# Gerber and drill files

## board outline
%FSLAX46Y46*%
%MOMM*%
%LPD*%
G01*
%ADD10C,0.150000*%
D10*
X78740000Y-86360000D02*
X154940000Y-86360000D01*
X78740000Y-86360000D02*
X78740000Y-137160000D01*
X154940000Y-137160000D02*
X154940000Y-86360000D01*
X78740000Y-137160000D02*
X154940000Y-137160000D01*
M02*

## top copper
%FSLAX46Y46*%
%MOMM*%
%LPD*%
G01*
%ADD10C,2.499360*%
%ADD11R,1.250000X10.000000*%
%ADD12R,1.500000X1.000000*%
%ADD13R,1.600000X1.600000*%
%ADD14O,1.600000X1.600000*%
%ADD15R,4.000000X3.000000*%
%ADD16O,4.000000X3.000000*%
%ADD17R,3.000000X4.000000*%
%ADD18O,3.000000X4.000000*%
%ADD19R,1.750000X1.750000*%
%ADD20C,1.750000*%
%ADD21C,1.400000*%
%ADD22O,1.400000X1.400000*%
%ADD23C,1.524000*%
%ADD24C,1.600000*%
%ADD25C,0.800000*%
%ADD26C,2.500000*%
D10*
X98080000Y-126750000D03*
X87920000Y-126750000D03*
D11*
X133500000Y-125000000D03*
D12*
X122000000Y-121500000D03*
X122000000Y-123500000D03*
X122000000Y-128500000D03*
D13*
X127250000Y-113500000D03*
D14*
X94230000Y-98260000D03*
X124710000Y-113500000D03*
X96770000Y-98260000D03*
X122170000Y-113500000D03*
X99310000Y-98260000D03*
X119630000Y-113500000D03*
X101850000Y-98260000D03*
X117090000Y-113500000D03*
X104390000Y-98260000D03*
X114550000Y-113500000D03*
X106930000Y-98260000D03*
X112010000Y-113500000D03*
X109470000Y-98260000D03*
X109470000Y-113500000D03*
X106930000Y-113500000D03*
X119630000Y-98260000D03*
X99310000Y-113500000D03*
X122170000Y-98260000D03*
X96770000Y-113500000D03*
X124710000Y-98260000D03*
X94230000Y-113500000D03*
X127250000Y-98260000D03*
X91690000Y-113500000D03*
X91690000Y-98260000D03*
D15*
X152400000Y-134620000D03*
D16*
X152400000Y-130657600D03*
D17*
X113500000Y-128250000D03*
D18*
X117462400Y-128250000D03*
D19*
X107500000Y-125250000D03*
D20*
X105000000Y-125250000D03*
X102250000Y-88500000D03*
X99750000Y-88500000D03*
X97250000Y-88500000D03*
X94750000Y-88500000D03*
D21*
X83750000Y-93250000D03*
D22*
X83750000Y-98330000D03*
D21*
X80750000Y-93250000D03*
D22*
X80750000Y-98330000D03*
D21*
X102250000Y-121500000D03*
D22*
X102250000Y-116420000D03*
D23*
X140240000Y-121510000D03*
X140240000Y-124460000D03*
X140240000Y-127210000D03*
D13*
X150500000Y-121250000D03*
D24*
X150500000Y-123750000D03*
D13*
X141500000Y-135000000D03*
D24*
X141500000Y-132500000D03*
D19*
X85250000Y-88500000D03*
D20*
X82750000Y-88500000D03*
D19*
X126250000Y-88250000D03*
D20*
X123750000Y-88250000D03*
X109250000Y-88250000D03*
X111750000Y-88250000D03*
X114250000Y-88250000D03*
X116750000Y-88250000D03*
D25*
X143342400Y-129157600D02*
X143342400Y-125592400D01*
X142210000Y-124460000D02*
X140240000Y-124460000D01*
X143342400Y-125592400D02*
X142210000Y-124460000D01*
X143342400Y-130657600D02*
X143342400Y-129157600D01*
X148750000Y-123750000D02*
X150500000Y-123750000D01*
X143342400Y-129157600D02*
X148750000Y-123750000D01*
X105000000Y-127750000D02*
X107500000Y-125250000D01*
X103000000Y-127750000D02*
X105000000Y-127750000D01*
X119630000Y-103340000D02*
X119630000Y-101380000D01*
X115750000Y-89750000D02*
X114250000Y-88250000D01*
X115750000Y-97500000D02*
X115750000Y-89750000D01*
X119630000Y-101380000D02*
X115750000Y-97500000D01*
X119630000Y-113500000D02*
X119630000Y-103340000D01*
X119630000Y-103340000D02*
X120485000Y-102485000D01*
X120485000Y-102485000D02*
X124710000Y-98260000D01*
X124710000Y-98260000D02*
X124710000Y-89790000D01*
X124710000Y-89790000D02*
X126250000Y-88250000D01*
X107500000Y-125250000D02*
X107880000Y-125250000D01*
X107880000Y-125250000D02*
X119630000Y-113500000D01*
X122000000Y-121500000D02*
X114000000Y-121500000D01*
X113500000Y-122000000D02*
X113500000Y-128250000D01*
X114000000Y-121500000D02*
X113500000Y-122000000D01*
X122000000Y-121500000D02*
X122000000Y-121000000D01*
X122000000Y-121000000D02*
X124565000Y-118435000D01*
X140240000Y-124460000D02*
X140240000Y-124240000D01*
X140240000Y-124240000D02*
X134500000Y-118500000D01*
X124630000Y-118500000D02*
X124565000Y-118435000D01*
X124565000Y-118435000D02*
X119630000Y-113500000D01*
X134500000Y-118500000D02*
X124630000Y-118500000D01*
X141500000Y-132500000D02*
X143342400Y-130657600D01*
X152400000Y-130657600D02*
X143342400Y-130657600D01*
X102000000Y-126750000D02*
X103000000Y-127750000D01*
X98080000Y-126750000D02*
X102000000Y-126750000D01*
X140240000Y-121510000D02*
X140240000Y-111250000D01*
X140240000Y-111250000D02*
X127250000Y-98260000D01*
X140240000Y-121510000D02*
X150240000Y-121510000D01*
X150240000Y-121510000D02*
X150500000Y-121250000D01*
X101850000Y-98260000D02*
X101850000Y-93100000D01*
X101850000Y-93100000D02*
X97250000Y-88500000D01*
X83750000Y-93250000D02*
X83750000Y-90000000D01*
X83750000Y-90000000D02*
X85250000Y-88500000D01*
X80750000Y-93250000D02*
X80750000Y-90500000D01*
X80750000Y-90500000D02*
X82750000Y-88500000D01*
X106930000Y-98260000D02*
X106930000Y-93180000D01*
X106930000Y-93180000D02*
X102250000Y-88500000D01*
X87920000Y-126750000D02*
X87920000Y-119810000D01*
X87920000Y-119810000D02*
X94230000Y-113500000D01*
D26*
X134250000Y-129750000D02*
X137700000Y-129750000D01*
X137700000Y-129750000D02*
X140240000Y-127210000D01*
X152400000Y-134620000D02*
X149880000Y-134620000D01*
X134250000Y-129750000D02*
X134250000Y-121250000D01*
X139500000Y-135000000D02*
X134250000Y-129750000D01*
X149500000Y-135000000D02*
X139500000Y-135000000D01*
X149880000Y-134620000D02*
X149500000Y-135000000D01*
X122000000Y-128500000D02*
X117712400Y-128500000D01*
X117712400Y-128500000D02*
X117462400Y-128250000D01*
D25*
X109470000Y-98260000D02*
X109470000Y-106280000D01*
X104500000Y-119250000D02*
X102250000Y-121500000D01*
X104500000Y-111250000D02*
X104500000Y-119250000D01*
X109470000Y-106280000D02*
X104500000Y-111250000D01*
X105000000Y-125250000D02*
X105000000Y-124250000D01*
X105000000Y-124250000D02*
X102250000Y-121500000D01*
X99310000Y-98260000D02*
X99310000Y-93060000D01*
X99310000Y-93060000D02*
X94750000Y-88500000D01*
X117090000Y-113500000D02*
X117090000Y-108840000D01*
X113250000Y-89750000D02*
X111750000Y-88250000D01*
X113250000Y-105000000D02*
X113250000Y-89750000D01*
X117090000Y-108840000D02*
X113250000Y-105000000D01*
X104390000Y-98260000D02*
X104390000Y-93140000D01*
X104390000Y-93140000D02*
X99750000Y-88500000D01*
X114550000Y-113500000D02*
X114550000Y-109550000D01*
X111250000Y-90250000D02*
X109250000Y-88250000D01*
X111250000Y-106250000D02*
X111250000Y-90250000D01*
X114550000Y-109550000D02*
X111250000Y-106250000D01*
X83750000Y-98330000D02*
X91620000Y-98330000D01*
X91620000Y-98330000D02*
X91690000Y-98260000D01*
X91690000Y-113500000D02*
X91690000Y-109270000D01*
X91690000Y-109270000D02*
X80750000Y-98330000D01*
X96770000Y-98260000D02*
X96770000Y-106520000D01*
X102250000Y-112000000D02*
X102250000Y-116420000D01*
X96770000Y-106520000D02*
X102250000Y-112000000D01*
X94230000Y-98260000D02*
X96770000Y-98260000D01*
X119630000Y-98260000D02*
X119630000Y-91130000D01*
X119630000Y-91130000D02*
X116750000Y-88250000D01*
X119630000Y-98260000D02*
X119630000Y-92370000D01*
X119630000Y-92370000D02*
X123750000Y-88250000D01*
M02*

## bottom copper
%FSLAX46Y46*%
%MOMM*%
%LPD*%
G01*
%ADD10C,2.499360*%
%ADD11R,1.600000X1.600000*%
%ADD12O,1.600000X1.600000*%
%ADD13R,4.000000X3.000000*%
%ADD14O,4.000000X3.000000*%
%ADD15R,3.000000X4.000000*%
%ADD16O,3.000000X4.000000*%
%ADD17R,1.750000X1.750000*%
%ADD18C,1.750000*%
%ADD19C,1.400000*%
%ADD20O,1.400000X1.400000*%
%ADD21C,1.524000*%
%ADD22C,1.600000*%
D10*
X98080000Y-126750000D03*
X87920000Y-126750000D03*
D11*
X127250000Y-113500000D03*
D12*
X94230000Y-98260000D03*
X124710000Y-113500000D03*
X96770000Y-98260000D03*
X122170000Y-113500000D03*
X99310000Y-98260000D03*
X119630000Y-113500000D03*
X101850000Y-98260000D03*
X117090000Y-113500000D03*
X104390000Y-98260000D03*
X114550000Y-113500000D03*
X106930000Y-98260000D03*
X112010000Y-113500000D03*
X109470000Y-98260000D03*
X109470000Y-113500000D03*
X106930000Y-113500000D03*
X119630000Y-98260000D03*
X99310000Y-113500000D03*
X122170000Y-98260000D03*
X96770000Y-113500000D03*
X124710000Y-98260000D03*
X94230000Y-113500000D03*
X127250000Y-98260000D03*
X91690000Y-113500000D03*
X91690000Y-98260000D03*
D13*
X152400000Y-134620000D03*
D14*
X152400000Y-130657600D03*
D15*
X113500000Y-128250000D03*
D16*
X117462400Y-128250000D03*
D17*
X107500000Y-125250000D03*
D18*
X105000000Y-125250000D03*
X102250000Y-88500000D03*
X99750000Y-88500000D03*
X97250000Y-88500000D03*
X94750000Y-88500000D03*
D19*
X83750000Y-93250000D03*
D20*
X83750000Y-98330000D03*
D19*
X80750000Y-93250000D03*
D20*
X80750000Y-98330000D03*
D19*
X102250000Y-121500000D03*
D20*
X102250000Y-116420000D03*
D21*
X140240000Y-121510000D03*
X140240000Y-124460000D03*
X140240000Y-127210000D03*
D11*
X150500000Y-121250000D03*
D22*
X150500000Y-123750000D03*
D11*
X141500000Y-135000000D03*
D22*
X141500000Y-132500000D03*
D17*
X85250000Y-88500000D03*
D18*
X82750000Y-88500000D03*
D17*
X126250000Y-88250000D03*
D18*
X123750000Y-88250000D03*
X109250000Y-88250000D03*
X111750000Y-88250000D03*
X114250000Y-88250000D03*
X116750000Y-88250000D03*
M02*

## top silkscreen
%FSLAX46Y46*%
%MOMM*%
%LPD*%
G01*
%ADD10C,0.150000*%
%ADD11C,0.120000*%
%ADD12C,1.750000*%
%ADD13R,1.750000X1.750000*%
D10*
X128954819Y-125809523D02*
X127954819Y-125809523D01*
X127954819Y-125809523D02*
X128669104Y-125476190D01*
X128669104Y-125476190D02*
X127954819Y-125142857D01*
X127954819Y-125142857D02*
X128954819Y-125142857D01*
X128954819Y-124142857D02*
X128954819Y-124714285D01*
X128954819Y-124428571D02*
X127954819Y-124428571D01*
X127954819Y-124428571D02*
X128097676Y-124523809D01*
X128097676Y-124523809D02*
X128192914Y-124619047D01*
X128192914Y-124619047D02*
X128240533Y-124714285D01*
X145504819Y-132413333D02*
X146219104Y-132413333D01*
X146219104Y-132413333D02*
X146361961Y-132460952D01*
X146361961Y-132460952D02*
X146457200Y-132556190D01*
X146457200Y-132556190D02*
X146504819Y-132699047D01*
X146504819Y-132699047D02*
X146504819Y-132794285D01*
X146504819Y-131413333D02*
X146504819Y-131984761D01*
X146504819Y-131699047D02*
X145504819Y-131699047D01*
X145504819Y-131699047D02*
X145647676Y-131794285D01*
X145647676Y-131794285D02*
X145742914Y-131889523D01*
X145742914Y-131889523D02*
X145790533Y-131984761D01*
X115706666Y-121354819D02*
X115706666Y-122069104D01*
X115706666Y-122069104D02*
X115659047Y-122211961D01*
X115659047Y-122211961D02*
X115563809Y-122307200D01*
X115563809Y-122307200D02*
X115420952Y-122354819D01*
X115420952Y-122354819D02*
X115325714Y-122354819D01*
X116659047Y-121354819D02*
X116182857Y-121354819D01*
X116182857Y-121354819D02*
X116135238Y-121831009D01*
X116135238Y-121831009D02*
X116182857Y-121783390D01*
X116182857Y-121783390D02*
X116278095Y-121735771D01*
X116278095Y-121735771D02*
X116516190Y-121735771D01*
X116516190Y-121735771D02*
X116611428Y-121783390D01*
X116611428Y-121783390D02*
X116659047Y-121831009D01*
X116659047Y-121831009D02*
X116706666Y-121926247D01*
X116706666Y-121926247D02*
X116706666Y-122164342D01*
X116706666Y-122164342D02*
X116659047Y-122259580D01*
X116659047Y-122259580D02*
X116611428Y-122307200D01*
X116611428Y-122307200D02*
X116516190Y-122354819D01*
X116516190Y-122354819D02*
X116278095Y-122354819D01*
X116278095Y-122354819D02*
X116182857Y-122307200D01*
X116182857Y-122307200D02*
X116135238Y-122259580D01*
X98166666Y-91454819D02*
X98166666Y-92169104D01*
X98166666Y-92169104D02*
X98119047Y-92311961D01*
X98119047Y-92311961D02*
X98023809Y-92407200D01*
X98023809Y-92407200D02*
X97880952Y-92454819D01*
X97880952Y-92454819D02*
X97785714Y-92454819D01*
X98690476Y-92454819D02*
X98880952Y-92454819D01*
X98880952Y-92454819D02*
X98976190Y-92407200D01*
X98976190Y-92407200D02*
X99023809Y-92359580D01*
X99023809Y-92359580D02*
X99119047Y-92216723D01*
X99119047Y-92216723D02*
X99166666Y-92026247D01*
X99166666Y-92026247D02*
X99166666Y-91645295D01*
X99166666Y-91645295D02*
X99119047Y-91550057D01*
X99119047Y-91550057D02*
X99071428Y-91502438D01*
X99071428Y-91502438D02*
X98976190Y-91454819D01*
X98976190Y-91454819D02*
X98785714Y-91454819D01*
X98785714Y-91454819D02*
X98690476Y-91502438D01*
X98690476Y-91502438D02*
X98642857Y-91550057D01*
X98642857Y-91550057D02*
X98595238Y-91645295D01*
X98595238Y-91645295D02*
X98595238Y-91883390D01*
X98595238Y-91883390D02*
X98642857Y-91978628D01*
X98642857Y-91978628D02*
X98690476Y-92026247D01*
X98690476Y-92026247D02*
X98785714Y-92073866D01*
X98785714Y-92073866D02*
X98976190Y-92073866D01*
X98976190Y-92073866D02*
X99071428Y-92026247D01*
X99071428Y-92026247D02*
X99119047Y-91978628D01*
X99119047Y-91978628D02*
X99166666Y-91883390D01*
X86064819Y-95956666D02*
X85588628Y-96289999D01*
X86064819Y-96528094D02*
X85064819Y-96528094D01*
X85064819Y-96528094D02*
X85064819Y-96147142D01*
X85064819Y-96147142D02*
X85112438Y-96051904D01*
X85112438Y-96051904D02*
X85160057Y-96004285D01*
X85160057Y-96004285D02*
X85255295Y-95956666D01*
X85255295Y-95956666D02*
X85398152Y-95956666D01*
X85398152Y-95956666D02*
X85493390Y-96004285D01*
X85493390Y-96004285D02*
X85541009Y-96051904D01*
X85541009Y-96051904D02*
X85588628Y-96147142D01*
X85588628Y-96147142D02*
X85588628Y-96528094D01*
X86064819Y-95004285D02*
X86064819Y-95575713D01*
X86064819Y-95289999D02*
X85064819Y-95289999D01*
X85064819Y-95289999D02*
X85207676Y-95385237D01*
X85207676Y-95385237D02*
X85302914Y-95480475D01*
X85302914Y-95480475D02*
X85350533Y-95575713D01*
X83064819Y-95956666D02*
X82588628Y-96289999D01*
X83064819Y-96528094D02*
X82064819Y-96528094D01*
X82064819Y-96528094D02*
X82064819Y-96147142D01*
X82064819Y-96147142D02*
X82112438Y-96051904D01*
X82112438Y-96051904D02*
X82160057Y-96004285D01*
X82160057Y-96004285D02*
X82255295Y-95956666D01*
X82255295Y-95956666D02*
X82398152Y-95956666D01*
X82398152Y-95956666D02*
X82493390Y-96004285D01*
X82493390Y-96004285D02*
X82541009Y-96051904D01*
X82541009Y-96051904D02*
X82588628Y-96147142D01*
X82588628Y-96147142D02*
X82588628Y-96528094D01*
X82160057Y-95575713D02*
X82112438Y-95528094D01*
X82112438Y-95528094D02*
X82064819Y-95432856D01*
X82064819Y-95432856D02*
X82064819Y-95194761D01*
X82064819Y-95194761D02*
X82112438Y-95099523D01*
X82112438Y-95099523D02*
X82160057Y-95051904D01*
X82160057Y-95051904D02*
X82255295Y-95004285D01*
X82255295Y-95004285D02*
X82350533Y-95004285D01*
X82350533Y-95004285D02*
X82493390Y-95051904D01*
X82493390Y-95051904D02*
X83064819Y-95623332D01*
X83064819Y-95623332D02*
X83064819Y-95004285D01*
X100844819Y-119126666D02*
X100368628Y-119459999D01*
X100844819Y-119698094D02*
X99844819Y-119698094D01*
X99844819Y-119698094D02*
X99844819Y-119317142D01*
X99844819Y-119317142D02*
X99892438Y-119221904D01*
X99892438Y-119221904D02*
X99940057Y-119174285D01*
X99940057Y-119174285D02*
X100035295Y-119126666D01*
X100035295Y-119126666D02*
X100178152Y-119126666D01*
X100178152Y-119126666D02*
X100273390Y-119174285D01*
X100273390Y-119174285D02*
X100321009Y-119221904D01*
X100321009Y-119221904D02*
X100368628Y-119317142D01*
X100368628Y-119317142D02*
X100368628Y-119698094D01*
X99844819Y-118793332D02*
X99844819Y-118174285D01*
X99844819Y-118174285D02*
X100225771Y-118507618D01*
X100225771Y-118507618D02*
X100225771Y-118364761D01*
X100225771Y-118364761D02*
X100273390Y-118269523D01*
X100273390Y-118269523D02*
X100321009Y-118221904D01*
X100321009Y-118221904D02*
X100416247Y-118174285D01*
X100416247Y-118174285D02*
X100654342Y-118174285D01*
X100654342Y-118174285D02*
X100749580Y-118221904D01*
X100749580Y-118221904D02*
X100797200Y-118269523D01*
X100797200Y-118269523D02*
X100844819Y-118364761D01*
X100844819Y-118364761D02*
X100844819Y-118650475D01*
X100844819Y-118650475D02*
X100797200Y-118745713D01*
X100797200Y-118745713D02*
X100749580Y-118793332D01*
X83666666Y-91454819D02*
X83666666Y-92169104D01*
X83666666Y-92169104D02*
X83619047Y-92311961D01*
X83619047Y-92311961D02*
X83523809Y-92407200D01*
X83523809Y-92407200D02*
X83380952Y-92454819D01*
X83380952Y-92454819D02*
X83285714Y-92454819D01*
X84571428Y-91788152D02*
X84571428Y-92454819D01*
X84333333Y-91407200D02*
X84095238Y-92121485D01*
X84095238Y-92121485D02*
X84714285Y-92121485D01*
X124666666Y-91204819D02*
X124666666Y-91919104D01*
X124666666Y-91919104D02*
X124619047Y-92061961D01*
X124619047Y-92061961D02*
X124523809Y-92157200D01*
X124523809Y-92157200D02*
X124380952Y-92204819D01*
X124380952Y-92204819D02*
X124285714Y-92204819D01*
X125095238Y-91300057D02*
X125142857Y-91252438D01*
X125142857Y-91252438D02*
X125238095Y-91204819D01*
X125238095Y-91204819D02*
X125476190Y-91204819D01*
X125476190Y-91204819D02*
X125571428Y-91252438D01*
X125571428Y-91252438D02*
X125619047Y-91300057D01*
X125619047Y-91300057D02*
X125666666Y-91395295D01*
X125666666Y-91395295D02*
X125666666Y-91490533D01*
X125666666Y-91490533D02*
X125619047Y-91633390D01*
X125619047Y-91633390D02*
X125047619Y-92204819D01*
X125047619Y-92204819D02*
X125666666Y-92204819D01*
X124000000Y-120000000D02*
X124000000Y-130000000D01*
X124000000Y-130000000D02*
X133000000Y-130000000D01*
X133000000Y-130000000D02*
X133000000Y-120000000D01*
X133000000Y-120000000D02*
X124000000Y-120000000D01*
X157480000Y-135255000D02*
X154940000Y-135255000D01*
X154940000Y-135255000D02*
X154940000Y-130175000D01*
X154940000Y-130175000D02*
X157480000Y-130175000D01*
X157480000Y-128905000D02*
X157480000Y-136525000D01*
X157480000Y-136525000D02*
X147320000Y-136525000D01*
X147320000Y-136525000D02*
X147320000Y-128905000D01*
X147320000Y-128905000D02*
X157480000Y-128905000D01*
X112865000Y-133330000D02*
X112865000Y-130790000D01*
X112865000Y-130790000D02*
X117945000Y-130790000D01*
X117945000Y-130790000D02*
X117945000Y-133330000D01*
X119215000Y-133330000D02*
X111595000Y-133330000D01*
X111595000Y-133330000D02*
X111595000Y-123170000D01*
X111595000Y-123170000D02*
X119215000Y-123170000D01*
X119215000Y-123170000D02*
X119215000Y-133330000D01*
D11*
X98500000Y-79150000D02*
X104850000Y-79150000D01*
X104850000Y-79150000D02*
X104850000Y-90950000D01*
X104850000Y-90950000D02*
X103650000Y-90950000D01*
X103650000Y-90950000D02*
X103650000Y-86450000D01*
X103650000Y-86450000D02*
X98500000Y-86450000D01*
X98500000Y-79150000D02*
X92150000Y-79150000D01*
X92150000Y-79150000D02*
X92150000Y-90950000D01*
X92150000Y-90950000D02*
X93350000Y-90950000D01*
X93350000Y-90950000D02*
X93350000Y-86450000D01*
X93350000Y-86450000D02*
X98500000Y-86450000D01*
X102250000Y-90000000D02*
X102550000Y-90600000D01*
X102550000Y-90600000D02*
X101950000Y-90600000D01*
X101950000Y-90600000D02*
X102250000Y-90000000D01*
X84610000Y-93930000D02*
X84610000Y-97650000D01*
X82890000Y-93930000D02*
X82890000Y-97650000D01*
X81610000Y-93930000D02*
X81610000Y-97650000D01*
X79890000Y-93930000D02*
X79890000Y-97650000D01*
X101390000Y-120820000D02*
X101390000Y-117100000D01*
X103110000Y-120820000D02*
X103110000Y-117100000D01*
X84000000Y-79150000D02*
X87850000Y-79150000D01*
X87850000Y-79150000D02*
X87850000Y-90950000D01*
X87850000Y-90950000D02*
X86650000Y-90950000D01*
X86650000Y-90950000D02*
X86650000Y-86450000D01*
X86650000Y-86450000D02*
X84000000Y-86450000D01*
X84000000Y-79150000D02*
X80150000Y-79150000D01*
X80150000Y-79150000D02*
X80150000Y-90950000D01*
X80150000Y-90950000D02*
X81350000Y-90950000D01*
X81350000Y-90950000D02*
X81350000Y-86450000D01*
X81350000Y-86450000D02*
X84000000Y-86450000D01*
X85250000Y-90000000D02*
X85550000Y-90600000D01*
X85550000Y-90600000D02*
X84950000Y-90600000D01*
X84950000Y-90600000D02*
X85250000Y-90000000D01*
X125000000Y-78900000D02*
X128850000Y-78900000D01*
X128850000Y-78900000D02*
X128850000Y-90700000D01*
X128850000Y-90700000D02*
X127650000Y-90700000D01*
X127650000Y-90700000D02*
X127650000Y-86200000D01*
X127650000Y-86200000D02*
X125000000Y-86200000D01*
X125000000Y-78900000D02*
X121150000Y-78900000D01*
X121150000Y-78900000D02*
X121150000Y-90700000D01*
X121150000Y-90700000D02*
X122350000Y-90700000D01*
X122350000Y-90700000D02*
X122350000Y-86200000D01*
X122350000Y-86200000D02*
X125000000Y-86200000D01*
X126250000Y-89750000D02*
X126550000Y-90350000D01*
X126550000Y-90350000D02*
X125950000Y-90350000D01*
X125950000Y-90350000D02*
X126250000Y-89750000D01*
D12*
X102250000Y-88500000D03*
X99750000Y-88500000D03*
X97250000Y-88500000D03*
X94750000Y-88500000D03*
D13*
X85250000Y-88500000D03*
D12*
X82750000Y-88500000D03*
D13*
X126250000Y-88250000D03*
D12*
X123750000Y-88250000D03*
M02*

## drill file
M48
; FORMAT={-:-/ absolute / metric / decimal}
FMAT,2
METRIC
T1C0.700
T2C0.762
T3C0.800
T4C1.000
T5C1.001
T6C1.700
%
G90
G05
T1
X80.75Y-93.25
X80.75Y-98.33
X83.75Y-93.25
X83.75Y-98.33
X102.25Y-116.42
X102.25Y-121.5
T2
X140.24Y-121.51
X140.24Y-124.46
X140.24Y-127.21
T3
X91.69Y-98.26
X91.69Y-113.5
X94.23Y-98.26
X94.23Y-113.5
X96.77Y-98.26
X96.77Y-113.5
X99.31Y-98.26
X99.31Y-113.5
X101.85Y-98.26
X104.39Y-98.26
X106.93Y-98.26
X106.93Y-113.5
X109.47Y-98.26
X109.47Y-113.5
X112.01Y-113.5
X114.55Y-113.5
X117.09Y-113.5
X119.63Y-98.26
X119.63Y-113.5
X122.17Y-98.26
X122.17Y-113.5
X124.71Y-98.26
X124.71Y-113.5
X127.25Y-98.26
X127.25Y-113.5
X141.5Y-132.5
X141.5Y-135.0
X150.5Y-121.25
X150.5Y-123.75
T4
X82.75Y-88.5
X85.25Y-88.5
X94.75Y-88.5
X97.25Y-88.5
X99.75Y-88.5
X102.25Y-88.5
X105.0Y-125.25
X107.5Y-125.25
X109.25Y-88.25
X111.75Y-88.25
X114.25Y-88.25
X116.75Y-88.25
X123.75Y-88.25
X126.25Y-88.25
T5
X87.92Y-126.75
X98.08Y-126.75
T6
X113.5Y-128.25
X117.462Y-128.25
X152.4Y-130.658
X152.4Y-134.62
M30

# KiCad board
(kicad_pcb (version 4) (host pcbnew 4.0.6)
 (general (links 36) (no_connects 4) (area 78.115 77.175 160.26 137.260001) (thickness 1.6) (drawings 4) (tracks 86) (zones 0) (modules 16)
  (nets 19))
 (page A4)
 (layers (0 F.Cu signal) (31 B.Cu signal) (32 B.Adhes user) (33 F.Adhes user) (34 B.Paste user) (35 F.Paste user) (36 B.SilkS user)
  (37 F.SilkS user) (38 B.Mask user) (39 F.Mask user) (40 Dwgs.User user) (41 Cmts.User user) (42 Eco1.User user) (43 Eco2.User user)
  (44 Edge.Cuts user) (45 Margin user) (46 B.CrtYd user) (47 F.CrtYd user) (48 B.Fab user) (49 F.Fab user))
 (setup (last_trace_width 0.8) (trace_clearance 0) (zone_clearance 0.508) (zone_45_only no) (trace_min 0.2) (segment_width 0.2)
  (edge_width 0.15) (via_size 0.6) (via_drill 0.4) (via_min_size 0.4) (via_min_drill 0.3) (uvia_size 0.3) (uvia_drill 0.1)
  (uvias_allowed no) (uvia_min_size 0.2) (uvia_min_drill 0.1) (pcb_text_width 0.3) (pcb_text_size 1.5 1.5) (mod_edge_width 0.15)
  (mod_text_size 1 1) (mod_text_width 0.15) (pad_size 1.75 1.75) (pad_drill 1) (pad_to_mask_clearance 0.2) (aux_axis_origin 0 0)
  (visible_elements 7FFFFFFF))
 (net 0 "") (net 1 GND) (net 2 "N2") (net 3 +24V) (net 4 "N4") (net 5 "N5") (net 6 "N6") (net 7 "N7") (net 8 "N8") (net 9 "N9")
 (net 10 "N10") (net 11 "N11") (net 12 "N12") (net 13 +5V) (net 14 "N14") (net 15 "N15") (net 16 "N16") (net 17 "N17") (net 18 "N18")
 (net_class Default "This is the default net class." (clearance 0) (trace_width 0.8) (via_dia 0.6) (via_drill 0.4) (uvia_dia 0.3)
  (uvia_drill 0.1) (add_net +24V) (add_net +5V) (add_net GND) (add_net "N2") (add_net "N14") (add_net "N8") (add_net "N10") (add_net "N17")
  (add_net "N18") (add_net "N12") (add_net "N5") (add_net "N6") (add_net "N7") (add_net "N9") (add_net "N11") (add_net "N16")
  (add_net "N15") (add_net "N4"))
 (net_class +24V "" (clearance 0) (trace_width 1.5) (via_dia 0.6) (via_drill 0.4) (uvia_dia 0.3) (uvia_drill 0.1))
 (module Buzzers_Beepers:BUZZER (layer B.Cu) (at 93 126.75)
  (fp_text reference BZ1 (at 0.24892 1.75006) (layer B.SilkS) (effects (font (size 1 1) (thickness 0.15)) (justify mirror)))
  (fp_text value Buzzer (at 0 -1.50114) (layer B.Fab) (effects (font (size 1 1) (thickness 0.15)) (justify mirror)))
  (pad 2 thru_hole circle (at 5.08 0) (size 2.49936 2.49936) (drill 1.00076) (layers *.Cu *.Mask) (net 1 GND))
  (pad 1 thru_hole circle (at -5.08 0) (size 2.49936 2.49936) (drill 1.00076) (layers *.Cu *.Mask) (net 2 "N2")))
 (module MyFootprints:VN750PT (layer F.Cu) (at 128 125 270)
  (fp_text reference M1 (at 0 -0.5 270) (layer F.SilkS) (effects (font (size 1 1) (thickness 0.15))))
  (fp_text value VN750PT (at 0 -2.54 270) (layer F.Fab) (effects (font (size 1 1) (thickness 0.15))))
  (fp_line (start -5 4) (end 5 4) (layer F.SilkS) (width 0.15))
  (fp_line (start 5 4) (end 5 -5) (layer F.SilkS) (width 0.15))
  (fp_line (start 5 -5) (end -5 -5) (layer F.SilkS) (width 0.15))
  (fp_line (start -5 -5) (end -5 4) (layer F.SilkS) (width 0.15))
  (pad Vcc smd rect (at 0 -5.5 270) (size 10 1.25) (layers F.Cu F.Paste F.Mask) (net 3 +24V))
  (pad GND smd rect (at -3.5 6 270) (size 1 1.5) (layers F.Cu F.Paste F.Mask) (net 1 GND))
  (pad Inpu smd rect (at -1.5 6 270) (size 1 1.5) (layers F.Cu F.Paste F.Mask) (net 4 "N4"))
  (pad Vout smd rect (at 3.5 6 270) (size 1 1.5) (layers F.Cu F.Paste F.Mask) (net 3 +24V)))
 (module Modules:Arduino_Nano (layer B.Cu) (at 127.25 113.5 90)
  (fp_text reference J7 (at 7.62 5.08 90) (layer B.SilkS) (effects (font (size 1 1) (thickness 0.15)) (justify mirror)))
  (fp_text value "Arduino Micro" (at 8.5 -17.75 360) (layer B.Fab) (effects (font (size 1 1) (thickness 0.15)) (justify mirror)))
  (pad TX thru_hole rect (at 0 0 90) (size 1.6 1.6) (drill 0.8) (layers *.Cu *.Mask))
  (pad 3.3V thru_hole oval (at 15.24 -33.02 90) (size 1.6 1.6) (drill 0.8) (layers *.Cu *.Mask) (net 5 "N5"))
  (pad RX thru_hole oval (at 0 -2.54 90) (size 1.6 1.6) (drill 0.8) (layers *.Cu *.Mask))
  (pad AREF thru_hole oval (at 15.24 -30.48 90) (size 1.6 1.6) (drill 0.8) (layers *.Cu *.Mask) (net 5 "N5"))
  (pad RS thru_hole oval (at 0 -5.08 90) (size 1.6 1.6) (drill 0.8) (layers *.Cu *.Mask))
  (pad A0 thru_hole oval (at 15.24 -27.94 90) (size 1.6 1.6) (drill 0.8) (layers *.Cu *.Mask) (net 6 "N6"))
  (pad GND thru_hole oval (at 0 -7.62 90) (size 1.6 1.6) (drill 0.8) (layers *.Cu *.Mask) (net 1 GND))
  (pad A1 thru_hole oval (at 15.24 -25.4 90) (size 1.6 1.6) (drill 0.8) (layers *.Cu *.Mask) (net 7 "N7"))
  (pad SDA thru_hole oval (at 0 -10.16 90) (size 1.6 1.6) (drill 0.8) (layers *.Cu *.Mask) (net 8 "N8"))
  (pad A2 thru_hole oval (at 15.24 -22.86 90) (size 1.6 1.6) (drill 0.8) (layers *.Cu *.Mask) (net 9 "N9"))
  (pad SCL thru_hole oval (at 0 -12.7 90) (size 1.6 1.6) (drill 0.8) (layers *.Cu *.Mask) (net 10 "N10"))
  (pad A3 thru_hole oval (at 15.24 -20.32 90) (size 1.6 1.6) (drill 0.8) (layers *.Cu *.Mask) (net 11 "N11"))
  (pad D4 thru_hole oval (at 0 -15.24 90) (size 1.6 1.6) (drill 0.8) (layers *.Cu *.Mask))
  (pad A4 thru_hole oval (at 15.24 -17.78 90) (size 1.6 1.6) (drill 0.8) (layers *.Cu *.Mask) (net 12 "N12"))
  (pad D5 thru_hole oval (at 0 -17.78 90) (size 1.6 1.6) (drill 0.8) (layers *.Cu *.Mask))
  (pad D6 thru_hole oval (at 0 -20.32 90) (size 1.6 1.6) (drill 0.8) (layers *.Cu *.Mask))
  (pad 5V thru_hole oval (at 15.24 -7.62 90) (size 1.6 1.6) (drill 0.8) (layers *.Cu *.Mask) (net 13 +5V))
  (pad D9 thru_hole oval (at 0 -27.94 90) (size 1.6 1.6) (drill 0.8) (layers *.Cu *.Mask))
  (pad RS thru_hole oval (at 15.24 -5.08 90) (size 1.6 1.6) (drill 0.8) (layers *.Cu *.Mask))
  (pad D10 thru_hole oval (at 0 -30.48 90) (size 1.6 1.6) (drill 0.8) (layers *.Cu *.Mask) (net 4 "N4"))
  (pad GND thru_hole oval (at 15.24 -2.54 90) (size 1.6 1.6) (drill 0.8) (layers *.Cu *.Mask) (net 1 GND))
  (pad D11 thru_hole oval (at 0 -33.02 90) (size 1.6 1.6) (drill 0.8) (layers *.Cu *.Mask) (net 2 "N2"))
  (pad Vin thru_hole oval (at 15.24 0 90) (size 1.6 1.6) (drill 0.8) (layers *.Cu *.Mask) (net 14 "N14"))
  (pad D12 thru_hole oval (at 0 -35.56 90) (size 1.6 1.6) (drill 0.8) (layers *.Cu *.Mask) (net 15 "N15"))
  (pad D13 thru_hole oval (at 15.24 -35.56 90) (size 1.6 1.6) (drill 0.8) (layers *.Cu *.Mask) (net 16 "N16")))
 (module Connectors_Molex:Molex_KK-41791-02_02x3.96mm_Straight (layer F.Cu) (at 152.4 134.62 90)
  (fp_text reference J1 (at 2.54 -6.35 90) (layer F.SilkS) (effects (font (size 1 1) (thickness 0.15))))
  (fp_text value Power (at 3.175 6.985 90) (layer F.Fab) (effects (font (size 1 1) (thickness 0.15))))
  (fp_line (start -0.635 5.08) (end -0.635 2.54) (layer F.SilkS) (width 0.15))
  (fp_line (start -0.635 2.54) (end 4.445 2.54) (layer F.SilkS) (width 0.15))
  (fp_line (start 4.445 2.54) (end 4.445 5.08) (layer F.SilkS) (width 0.15))
  (fp_line (start 5.715 5.08) (end -1.905 5.08) (layer F.SilkS) (width 0.15))
  (fp_line (start -1.905 5.08) (end -1.905 -5.08) (layer F.SilkS) (width 0.15))
  (fp_line (start -1.905 -5.08) (end 5.715 -5.08) (layer F.SilkS) (width 0.15))
  (fp_line (start 5.715 -5.08) (end 5.715 5.08) (layer F.SilkS) (width 0.15))
  (pad 1 thru_hole rect (at 0 0 90) (size 3 4) (drill 1.7) (layers *.Cu *.Mask) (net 3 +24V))
  (pad 2 thru_hole oval (at 3.9624 0 90) (size 3 4) (drill 1.7) (layers *.Cu *.Mask) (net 1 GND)))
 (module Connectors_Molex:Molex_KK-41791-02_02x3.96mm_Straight (layer F.Cu) (at 113.5 128.25)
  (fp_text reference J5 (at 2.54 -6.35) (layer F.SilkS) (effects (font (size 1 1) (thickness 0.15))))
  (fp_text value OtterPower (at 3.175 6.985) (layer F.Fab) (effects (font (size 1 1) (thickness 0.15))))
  (fp_line (start -0.635 5.08) (end -0.635 2.54) (layer F.SilkS) (width 0.15))
  (fp_line (start -0.635 2.54) (end 4.445 2.54) (layer F.SilkS) (width 0.15))
  (fp_line (start 4.445 2.54) (end 4.445 5.08) (layer F.SilkS) (width 0.15))
  (fp_line (start 5.715 5.08) (end -1.905 5.08) (layer F.SilkS) (width 0.15))
  (fp_line (start -1.905 5.08) (end -1.905 -5.08) (layer F.SilkS) (width 0.15))
  (fp_line (start -1.905 -5.08) (end 5.715 -5.08) (layer F.SilkS) (width 0.15))
  (fp_line (start 5.715 -5.08) (end 5.715 5.08) (layer F.SilkS) (width 0.15))
  (pad 1 thru_hole rect (at 0 0) (size 3 4) (drill 1.7) (layers *.Cu *.Mask) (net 1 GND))
  (pad 2 thru_hole oval (at 3.9624 0) (size 3 4) (drill 1.7) (layers *.Cu *.Mask) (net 3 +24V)))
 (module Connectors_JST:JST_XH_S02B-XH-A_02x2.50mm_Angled (layer B.Cu) (at 107.5 125.25 180)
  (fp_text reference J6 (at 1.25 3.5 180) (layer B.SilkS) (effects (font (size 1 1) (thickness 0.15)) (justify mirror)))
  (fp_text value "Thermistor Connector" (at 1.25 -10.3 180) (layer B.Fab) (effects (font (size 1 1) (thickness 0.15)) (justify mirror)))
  (pad 1 thru_hole rect (at 0 0 180) (size 1.75 1.75) (drill 1) (layers *.Cu *.Mask B.SilkS) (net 1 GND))
  (pad 2 thru_hole circle (at 2.5 0 180) (size 1.75 1.75) (drill 1) (layers *.Cu *.Mask B.SilkS) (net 12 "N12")))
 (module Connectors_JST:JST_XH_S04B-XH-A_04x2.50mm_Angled (layer F.Cu) (at 102.25 88.5 180)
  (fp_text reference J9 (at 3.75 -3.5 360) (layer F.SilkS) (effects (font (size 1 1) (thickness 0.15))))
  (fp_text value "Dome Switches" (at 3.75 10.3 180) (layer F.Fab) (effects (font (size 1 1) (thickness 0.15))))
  (fp_line (start 3.75 9.35) (end -2.6 9.35) (layer F.SilkS) (width 0.12))
  (fp_line (start -2.6 9.35) (end -2.6 -2.45) (layer F.SilkS) (width 0.12))
  (fp_line (start -2.6 -2.45) (end -1.4 -2.45) (layer F.SilkS) (width 0.12))
  (fp_line (start -1.4 -2.45) (end -1.4 2.05) (layer F.SilkS) (width 0.12))
  (fp_line (start -1.4 2.05) (end 3.75 2.05) (layer F.SilkS) (width 0.12))
  (fp_line (start 3.75 9.35) (end 10.1 9.35) (layer F.SilkS) (width 0.12))
  (fp_line (start 10.1 9.35) (end 10.1 -2.45) (layer F.SilkS) (width 0.12))
  (fp_line (start 10.1 -2.45) (end 8.9 -2.45) (layer F.SilkS) (width 0.12))
  (fp_line (start 8.9 -2.45) (end 8.9 2.05) (layer F.SilkS) (width 0.12))
  (fp_line (start 8.9 2.05) (end 3.75 2.05) (layer F.SilkS) (width 0.12))
  (fp_line (start 0 -1.5) (end -0.3 -2.1) (layer F.SilkS) (width 0.12))
  (fp_line (start -0.3 -2.1) (end 0.3 -2.1) (layer F.SilkS) (width 0.12))
  (fp_line (start 0.3 -2.1) (end 0 -1.5) (layer F.SilkS) (width 0.12))
  (pad 1 thru_hole circle (at 0 0 180) (size 1.75 1.75) (drill 1) (layers *.Cu *.Mask F.SilkS) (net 11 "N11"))
  (pad 2 thru_hole circle (at 2.5 0 180) (size 1.75 1.75) (drill 1) (layers *.Cu *.Mask F.SilkS) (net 9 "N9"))
  (pad 3 thru_hole circle (at 5 0 180) (size 1.75 1.75) (drill 1) (layers *.Cu *.Mask F.SilkS) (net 7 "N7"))
  (pad 4 thru_hole circle (at 7.5 0 180) (size 1.75 1.75) (drill 1) (layers *.Cu *.Mask F.SilkS) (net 6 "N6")))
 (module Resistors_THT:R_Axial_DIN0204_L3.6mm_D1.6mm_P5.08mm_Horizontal (layer F.Cu) (at 83.75 93.25 270)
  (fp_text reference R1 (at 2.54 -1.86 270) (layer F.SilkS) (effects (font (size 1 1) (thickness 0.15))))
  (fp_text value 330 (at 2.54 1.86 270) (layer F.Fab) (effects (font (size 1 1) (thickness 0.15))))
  (fp_line (start 0.68 -0.86) (end 4.4 -0.86) (layer F.SilkS) (width 0.12))
  (fp_line (start 0.68 0.86) (end 4.4 0.86) (layer F.SilkS) (width 0.12))
  (pad 1 thru_hole circle (at 0 0 270) (size 1.4 1.4) (drill 0.7) (layers *.Cu *.Mask) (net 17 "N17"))
  (pad 2 thru_hole oval (at 5.08 0 270) (size 1.4 1.4) (drill 0.7) (layers *.Cu *.Mask) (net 16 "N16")))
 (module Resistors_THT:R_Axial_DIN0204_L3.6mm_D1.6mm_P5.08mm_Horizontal (layer F.Cu) (at 80.75 93.25 270)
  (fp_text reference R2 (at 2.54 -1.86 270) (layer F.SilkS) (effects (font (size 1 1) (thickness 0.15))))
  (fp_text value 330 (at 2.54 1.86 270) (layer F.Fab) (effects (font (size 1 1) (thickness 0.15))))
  (fp_line (start 0.68 -0.86) (end 4.4 -0.86) (layer F.SilkS) (width 0.12))
  (fp_line (start 0.68 0.86) (end 4.4 0.86) (layer F.SilkS) (width 0.12))
  (pad 1 thru_hole circle (at 0 0 270) (size 1.4 1.4) (drill 0.7) (layers *.Cu *.Mask) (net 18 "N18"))
  (pad 2 thru_hole oval (at 5.08 0 270) (size 1.4 1.4) (drill 0.7) (layers *.Cu *.Mask) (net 15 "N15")))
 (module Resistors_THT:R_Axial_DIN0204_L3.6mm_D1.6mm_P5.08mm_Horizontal (layer F.Cu) (at 102.25 121.5 90)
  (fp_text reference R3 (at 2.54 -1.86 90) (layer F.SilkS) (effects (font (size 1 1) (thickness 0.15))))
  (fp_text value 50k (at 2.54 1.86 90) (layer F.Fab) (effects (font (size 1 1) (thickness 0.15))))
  (fp_line (start 0.68 -0.86) (end 4.4 -0.86) (layer F.SilkS) (width 0.12))
  (fp_line (start 0.68 0.86) (end 4.4 0.86) (layer F.SilkS) (width 0.12))
  (pad 1 thru_hole circle (at 0 0 90) (size 1.4 1.4) (drill 0.7) (layers *.Cu *.Mask) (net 12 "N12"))
  (pad 2 thru_hole oval (at 5.08 0 90) (size 1.4 1.4) (drill 0.7) (layers *.Cu *.Mask) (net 5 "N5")))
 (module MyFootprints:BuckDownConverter (layer B.Cu) (at 142.24 124.46 270)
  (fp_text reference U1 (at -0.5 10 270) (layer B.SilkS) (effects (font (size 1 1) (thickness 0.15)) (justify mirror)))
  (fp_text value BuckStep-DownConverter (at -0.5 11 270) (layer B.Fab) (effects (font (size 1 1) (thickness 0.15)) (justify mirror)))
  (pad Vout thru_hole circle (at -2.95 2 270) (size 1.524 1.524) (drill 0.762) (layers *.Cu *.Mask) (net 14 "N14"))
  (pad GND thru_hole circle (at 0 2 270) (size 1.524 1.524) (drill 0.762) (layers *.Cu *.Mask) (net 1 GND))
  (pad Vin thru_hole circle (at 2.75 2 270) (size 1.524 1.524) (drill 0.762) (layers *.Cu *.Mask) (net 3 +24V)))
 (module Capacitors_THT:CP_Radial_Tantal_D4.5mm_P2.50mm (layer B.Cu) (at 150.5 121.25 270)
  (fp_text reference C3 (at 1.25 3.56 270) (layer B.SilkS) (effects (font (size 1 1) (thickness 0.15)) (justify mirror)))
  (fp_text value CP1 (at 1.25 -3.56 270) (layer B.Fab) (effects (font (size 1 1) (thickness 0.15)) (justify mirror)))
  (pad 1 thru_hole rect (at 0 0 270) (size 1.6 1.6) (drill 0.8) (layers *.Cu *.Mask) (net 14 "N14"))
  (pad 2 thru_hole circle (at 2.5 0 270) (size 1.6 1.6) (drill 0.8) (layers *.Cu *.Mask) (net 1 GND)))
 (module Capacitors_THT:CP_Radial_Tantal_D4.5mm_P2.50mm (layer B.Cu) (at 141.5 135 90)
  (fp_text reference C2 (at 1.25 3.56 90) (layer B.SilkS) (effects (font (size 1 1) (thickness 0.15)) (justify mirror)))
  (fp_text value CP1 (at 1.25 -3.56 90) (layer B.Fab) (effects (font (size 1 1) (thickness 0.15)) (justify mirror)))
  (pad 1 thru_hole rect (at 0 0 90) (size 1.6 1.6) (drill 0.8) (layers *.Cu *.Mask) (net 3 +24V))
  (pad 2 thru_hole circle (at 2.5 0 90) (size 1.6 1.6) (drill 0.8) (layers *.Cu *.Mask) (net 1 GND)))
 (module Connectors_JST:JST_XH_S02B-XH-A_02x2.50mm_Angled (layer F.Cu) (at 85.25 88.5 180)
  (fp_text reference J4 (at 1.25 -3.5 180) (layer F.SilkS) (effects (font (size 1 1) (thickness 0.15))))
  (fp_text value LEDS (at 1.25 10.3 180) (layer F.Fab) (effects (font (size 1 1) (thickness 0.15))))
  (fp_line (start 1.25 9.35) (end -2.6 9.35) (layer F.SilkS) (width 0.12))
  (fp_line (start -2.6 9.35) (end -2.6 -2.45) (layer F.SilkS) (width 0.12))
  (fp_line (start -2.6 -2.45) (end -1.4 -2.45) (layer F.SilkS) (width 0.12))
  (fp_line (start -1.4 -2.45) (end -1.4 2.05) (layer F.SilkS) (width 0.12))
  (fp_line (start -1.4 2.05) (end 1.25 2.05) (layer F.SilkS) (width 0.12))
  (fp_line (start 1.25 9.35) (end 5.1 9.35) (layer F.SilkS) (width 0.12))
  (fp_line (start 5.1 9.35) (end 5.1 -2.45) (layer F.SilkS) (width 0.12))
  (fp_line (start 5.1 -2.45) (end 3.9 -2.45) (layer F.SilkS) (width 0.12))
  (fp_line (start 3.9 -2.45) (end 3.9 2.05) (layer F.SilkS) (width 0.12))
  (fp_line (start 3.9 2.05) (end 1.25 2.05) (layer F.SilkS) (width 0.12))
  (fp_line (start 0 -1.5) (end -0.3 -2.1) (layer F.SilkS) (width 0.12))
  (fp_line (start -0.3 -2.1) (end 0.3 -2.1) (layer F.SilkS) (width 0.12))
  (fp_line (start 0.3 -2.1) (end 0 -1.5) (layer F.SilkS) (width 0.12))
  (pad 1 thru_hole rect (at 0 0 180) (size 1.75 1.75) (drill 1) (layers *.Cu *.Mask F.SilkS) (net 17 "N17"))
  (pad 2 thru_hole circle (at 2.5 0 180) (size 1.75 1.75) (drill 1) (layers *.Cu *.Mask F.SilkS) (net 18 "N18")))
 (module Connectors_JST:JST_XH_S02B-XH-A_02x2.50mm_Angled (layer F.Cu) (at 126.25 88.25 180)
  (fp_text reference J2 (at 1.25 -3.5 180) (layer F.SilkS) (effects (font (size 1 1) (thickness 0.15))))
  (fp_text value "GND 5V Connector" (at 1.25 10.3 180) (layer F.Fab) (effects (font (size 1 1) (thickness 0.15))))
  (fp_line (start 1.25 9.35) (end -2.6 9.35) (layer F.SilkS) (width 0.12))
  (fp_line (start -2.6 9.35) (end -2.6 -2.45) (layer F.SilkS) (width 0.12))
  (fp_line (start -2.6 -2.45) (end -1.4 -2.45) (layer F.SilkS) (width 0.12))
  (fp_line (start -1.4 -2.45) (end -1.4 2.05) (layer F.SilkS) (width 0.12))
  (fp_line (start -1.4 2.05) (end 1.25 2.05) (layer F.SilkS) (width 0.12))
  (fp_line (start 1.25 9.35) (end 5.1 9.35) (layer F.SilkS) (width 0.12))
  (fp_line (start 5.1 9.35) (end 5.1 -2.45) (layer F.SilkS) (width 0.12))
  (fp_line (start 5.1 -2.45) (end 3.9 -2.45) (layer F.SilkS) (width 0.12))
  (fp_line (start 3.9 -2.45) (end 3.9 2.05) (layer F.SilkS) (width 0.12))
  (fp_line (start 3.9 2.05) (end 1.25 2.05) (layer F.SilkS) (width 0.12))
  (fp_line (start 0 -1.5) (end -0.3 -2.1) (layer F.SilkS) (width 0.12))
  (fp_line (start -0.3 -2.1) (end 0.3 -2.1) (layer F.SilkS) (width 0.12))
  (fp_line (start 0.3 -2.1) (end 0 -1.5) (layer F.SilkS) (width 0.12))
  (pad 1 thru_hole rect (at 0 0 180) (size 1.75 1.75) (drill 1) (layers *.Cu *.Mask F.SilkS) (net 1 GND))
  (pad 2 thru_hole circle (at 2.5 0 180) (size 1.75 1.75) (drill 1) (layers *.Cu *.Mask F.SilkS) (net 13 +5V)))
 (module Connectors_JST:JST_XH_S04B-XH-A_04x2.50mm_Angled (layer B.Cu) (at 109.25 88.25)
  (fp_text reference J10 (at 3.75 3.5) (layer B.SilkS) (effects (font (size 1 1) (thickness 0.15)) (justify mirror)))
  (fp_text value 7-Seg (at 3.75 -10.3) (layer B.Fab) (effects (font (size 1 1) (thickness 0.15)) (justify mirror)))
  (pad 1 thru_hole circle (at 0 0) (size 1.75 1.75) (drill 1) (layers *.Cu *.Mask B.SilkS) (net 10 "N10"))
  (pad 2 thru_hole circle (at 2.5 0) (size 1.75 1.75) (drill 1) (layers *.Cu *.Mask B.SilkS) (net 8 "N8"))
  (pad 3 thru_hole circle (at 5 0) (size 1.75 1.75) (drill 1) (layers *.Cu *.Mask B.SilkS) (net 1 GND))
  (pad 4 thru_hole circle (at 7.5 0) (size 1.75 1.75) (drill 1) (layers *.Cu *.Mask B.SilkS) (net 13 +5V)))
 (gr_line (start 78.74 86.36) (end 154.94 86.36) (angle 90) (layer Edge.Cuts) (width 0.15))
 (gr_line (start 78.74 86.36) (end 78.74 137.16) (angle 90) (layer Edge.Cuts) (width 0.15))
 (gr_line (start 154.94 137.16) (end 154.94 86.36) (angle 90) (layer Edge.Cuts) (width 0.15))
 (gr_line (start 78.74 137.16) (end 154.94 137.16) (angle 90) (layer Edge.Cuts) (width 0.15))
 (segment (start 143.3424 129.1576) (end 143.3424 125.5924) (width 0.8) (layer F.Cu) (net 1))
 (segment (start 142.21 124.46) (end 140.24 124.46) (width 0.8) (layer F.Cu) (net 1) (status 800000))
 (segment (start 143.3424 125.5924) (end 142.21 124.46) (width 0.8) (layer F.Cu) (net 1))
 (segment (start 143.3424 130.6576) (end 143.3424 129.1576) (width 0.8) (layer F.Cu) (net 1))
 (segment (start 148.75 123.75) (end 150.5 123.75) (width 0.8) (layer F.Cu) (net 1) (status 800000))
 (segment (start 143.3424 129.1576) (end 148.75 123.75) (width 0.8) (layer F.Cu) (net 1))
 (segment (start 105 127.75) (end 107.5 125.25) (width 0.8) (layer F.Cu) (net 1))
 (segment (start 103 127.75) (end 105 127.75) (width 0.8) (layer F.Cu) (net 1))
 (segment (start 119.63 103.34) (end 119.63 101.38) (width 0.8) (layer F.Cu) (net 1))
 (segment (start 115.75 89.75) (end 114.25 88.25) (width 0.8) (layer F.Cu) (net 1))
 (segment (start 115.75 97.5) (end 115.75 89.75) (width 0.8) (layer F.Cu) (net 1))
 (segment (start 119.63 101.38) (end 115.75 97.5) (width 0.8) (layer F.Cu) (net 1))
 (segment (start 119.63 113.5) (end 119.63 103.34) (width 0.8) (layer F.Cu) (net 1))
 (segment (start 119.63 103.34) (end 120.485 102.485) (width 0.8) (layer F.Cu) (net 1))
 (segment (start 120.485 102.485) (end 124.71 98.26) (width 0.8) (layer F.Cu) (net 1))
 (segment (start 124.71 98.26) (end 124.71 89.79) (width 0.8) (layer F.Cu) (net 1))
 (segment (start 124.71 89.79) (end 126.25 88.25) (width 0.8) (layer F.Cu) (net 1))
 (segment (start 107.5 125.25) (end 107.88 125.25) (width 0.8) (layer F.Cu) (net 1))
 (segment (start 107.88 125.25) (end 119.63 113.5) (width 0.8) (layer F.Cu) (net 1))
 (segment (start 122 121.5) (end 114 121.5) (width 0.8) (layer F.Cu) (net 1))
 (segment (start 113.5 122) (end 113.5 128.25) (width 0.8) (layer F.Cu) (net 1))
 (segment (start 114 121.5) (end 113.5 122) (width 0.8) (layer F.Cu) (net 1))
 (segment (start 122 121.5) (end 122 121) (width 0.8) (layer F.Cu) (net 1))
 (segment (start 122 121) (end 124.565 118.435) (width 0.8) (layer F.Cu) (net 1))
 (segment (start 140.24 124.46) (end 140.24 124.24) (width 0.8) (layer F.Cu) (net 1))
 (segment (start 140.24 124.24) (end 134.5 118.5) (width 0.8) (layer F.Cu) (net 1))
 (segment (start 124.63 118.5) (end 124.565 118.435) (width 0.8) (layer F.Cu) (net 1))
 (segment (start 124.565 118.435) (end 119.63 113.5) (width 0.8) (layer F.Cu) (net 1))
 (segment (start 134.5 118.5) (end 124.63 118.5) (width 0.8) (layer F.Cu) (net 1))
 (segment (start 141.5 132.5) (end 143.3424 130.6576) (width 0.8) (layer F.Cu) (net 1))
 (segment (start 152.4 130.6576) (end 143.3424 130.6576) (width 0.8) (layer F.Cu) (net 1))
 (segment (start 102 126.75) (end 103 127.75) (width 0.8) (layer F.Cu) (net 1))
 (segment (start 98.08 126.75) (end 102 126.75) (width 0.8) (layer F.Cu) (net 1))
 (segment (start 140.24 121.51) (end 140.24 111.25) (width 0.8) (layer F.Cu) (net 14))
 (segment (start 140.24 111.25) (end 127.25 98.26) (width 0.8) (layer F.Cu) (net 14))
 (segment (start 140.24 121.51) (end 150.24 121.51) (width 0.8) (layer F.Cu) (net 14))
 (segment (start 150.24 121.51) (end 150.5 121.25) (width 0.8) (layer F.Cu) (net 14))
 (segment (start 101.85 98.26) (end 101.85 93.1) (width 0.8) (layer F.Cu) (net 7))
 (segment (start 101.85 93.1) (end 97.25 88.5) (width 0.8) (layer F.Cu) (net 7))
 (segment (start 83.75 93.25) (end 83.75 90) (width 0.8) (layer F.Cu) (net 17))
 (segment (start 83.75 90) (end 85.25 88.5) (width 0.8) (layer F.Cu) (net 17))
 (segment (start 80.75 93.25) (end 80.75 90.5) (width 0.8) (layer F.Cu) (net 18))
 (segment (start 80.75 90.5) (end 82.75 88.5) (width 0.8) (layer F.Cu) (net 18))
 (segment (start 106.93 98.26) (end 106.93 93.18) (width 0.8) (layer F.Cu) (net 11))
 (segment (start 106.93 93.18) (end 102.25 88.5) (width 0.8) (layer F.Cu) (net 11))
 (segment (start 87.92 126.75) (end 87.92 119.81) (width 0.8) (layer F.Cu) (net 2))
 (segment (start 87.92 119.81) (end 94.23 113.5) (width 0.8) (layer F.Cu) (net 2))
 (segment (start 134.25 129.75) (end 137.7 129.75) (width 2.5) (layer F.Cu) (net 3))
 (segment (start 137.7 129.75) (end 140.24 127.21) (width 2.5) (layer F.Cu) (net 3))
 (segment (start 152.4 134.62) (end 149.88 134.62) (width 2.5) (layer F.Cu) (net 3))
 (segment (start 134.25 129.75) (end 134.25 121.25) (width 2.5) (layer F.Cu) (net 3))
 (segment (start 139.5 135) (end 134.25 129.75) (width 2.5) (layer F.Cu) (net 3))
 (segment (start 149.5 135) (end 139.5 135) (width 2.5) (layer F.Cu) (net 3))
 (segment (start 149.88 134.62) (end 149.5 135) (width 2.5) (layer F.Cu) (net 3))
 (segment (start 122 128.5) (end 117.7124 128.5) (width 2.5) (layer F.Cu) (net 3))
 (segment (start 117.7124 128.5) (end 117.4624 128.25) (width 2.5) (layer F.Cu) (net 3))
 (segment (start 109.47 98.26) (end 109.47 106.28) (width 0.8) (layer F.Cu) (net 12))
 (segment (start 104.5 119.25) (end 102.25 121.5) (width 0.8) (layer F.Cu) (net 12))
 (segment (start 104.5 111.25) (end 104.5 119.25) (width 0.8) (layer F.Cu) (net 12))
 (segment (start 109.47 106.28) (end 104.5 111.25) (width 0.8) (layer F.Cu) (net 12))
 (segment (start 105 125.25) (end 105 124.25) (width 0.8) (layer F.Cu) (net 12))
 (segment (start 105 124.25) (end 102.25 121.5) (width 0.8) (layer F.Cu) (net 12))
 (segment (start 99.31 98.26) (end 99.31 93.06) (width 0.8) (layer F.Cu) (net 6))
 (segment (start 99.31 93.06) (end 94.75 88.5) (width 0.8) (layer F.Cu) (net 6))
 (segment (start 117.09 113.5) (end 117.09 108.84) (width 0.8) (layer F.Cu) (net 8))
 (segment (start 113.25 89.75) (end 111.75 88.25) (width 0.8) (layer F.Cu) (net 8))
 (segment (start 113.25 105) (end 113.25 89.75) (width 0.8) (layer F.Cu) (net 8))
 (segment (start 117.09 108.84) (end 113.25 105) (width 0.8) (layer F.Cu) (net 8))
 (segment (start 104.39 98.26) (end 104.39 93.14) (width 0.8) (layer F.Cu) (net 9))
 (segment (start 104.39 93.14) (end 99.75 88.5) (width 0.8) (layer F.Cu) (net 9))
 (segment (start 114.55 113.5) (end 114.55 109.55) (width 0.8) (layer F.Cu) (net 10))
 (segment (start 111.25 90.25) (end 109.25 88.25) (width 0.8) (layer F.Cu) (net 10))
 (segment (start 111.25 106.25) (end 111.25 90.25) (width 0.8) (layer F.Cu) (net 10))
 (segment (start 114.55 109.55) (end 111.25 106.25) (width 0.8) (layer F.Cu) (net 10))
 (segment (start 83.75 98.33) (end 91.62 98.33) (width 0.8) (layer F.Cu) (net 16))
 (segment (start 91.62 98.33) (end 91.69 98.26) (width 0.8) (layer F.Cu) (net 16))
 (segment (start 91.69 113.5) (end 91.69 109.27) (width 0.8) (layer F.Cu) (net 15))
 (segment (start 91.69 109.27) (end 80.75 98.33) (width 0.8) (layer F.Cu) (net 15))
 (segment (start 96.77 98.26) (end 96.77 106.52) (width 0.8) (layer F.Cu) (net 5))
 (segment (start 102.25 112) (end 102.25 116.42) (width 0.8) (layer F.Cu) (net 5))
 (segment (start 96.77 106.52) (end 102.25 112) (width 0.8) (layer F.Cu) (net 5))
 (segment (start 94.23 98.26) (end 96.77 98.26) (width 0.8) (layer F.Cu) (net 5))
 (segment (start 119.63 98.26) (end 119.63 91.13) (width 0.8) (layer F.Cu) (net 13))
 (segment (start 119.63 91.13) (end 116.75 88.25) (width 0.8) (layer F.Cu) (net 13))
 (segment (start 119.63 98.26) (end 119.63 92.37) (width 0.8) (layer F.Cu) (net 13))
 (segment (start 119.63 92.37) (end 123.75 88.25) (width 0.8) (layer F.Cu) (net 13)))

